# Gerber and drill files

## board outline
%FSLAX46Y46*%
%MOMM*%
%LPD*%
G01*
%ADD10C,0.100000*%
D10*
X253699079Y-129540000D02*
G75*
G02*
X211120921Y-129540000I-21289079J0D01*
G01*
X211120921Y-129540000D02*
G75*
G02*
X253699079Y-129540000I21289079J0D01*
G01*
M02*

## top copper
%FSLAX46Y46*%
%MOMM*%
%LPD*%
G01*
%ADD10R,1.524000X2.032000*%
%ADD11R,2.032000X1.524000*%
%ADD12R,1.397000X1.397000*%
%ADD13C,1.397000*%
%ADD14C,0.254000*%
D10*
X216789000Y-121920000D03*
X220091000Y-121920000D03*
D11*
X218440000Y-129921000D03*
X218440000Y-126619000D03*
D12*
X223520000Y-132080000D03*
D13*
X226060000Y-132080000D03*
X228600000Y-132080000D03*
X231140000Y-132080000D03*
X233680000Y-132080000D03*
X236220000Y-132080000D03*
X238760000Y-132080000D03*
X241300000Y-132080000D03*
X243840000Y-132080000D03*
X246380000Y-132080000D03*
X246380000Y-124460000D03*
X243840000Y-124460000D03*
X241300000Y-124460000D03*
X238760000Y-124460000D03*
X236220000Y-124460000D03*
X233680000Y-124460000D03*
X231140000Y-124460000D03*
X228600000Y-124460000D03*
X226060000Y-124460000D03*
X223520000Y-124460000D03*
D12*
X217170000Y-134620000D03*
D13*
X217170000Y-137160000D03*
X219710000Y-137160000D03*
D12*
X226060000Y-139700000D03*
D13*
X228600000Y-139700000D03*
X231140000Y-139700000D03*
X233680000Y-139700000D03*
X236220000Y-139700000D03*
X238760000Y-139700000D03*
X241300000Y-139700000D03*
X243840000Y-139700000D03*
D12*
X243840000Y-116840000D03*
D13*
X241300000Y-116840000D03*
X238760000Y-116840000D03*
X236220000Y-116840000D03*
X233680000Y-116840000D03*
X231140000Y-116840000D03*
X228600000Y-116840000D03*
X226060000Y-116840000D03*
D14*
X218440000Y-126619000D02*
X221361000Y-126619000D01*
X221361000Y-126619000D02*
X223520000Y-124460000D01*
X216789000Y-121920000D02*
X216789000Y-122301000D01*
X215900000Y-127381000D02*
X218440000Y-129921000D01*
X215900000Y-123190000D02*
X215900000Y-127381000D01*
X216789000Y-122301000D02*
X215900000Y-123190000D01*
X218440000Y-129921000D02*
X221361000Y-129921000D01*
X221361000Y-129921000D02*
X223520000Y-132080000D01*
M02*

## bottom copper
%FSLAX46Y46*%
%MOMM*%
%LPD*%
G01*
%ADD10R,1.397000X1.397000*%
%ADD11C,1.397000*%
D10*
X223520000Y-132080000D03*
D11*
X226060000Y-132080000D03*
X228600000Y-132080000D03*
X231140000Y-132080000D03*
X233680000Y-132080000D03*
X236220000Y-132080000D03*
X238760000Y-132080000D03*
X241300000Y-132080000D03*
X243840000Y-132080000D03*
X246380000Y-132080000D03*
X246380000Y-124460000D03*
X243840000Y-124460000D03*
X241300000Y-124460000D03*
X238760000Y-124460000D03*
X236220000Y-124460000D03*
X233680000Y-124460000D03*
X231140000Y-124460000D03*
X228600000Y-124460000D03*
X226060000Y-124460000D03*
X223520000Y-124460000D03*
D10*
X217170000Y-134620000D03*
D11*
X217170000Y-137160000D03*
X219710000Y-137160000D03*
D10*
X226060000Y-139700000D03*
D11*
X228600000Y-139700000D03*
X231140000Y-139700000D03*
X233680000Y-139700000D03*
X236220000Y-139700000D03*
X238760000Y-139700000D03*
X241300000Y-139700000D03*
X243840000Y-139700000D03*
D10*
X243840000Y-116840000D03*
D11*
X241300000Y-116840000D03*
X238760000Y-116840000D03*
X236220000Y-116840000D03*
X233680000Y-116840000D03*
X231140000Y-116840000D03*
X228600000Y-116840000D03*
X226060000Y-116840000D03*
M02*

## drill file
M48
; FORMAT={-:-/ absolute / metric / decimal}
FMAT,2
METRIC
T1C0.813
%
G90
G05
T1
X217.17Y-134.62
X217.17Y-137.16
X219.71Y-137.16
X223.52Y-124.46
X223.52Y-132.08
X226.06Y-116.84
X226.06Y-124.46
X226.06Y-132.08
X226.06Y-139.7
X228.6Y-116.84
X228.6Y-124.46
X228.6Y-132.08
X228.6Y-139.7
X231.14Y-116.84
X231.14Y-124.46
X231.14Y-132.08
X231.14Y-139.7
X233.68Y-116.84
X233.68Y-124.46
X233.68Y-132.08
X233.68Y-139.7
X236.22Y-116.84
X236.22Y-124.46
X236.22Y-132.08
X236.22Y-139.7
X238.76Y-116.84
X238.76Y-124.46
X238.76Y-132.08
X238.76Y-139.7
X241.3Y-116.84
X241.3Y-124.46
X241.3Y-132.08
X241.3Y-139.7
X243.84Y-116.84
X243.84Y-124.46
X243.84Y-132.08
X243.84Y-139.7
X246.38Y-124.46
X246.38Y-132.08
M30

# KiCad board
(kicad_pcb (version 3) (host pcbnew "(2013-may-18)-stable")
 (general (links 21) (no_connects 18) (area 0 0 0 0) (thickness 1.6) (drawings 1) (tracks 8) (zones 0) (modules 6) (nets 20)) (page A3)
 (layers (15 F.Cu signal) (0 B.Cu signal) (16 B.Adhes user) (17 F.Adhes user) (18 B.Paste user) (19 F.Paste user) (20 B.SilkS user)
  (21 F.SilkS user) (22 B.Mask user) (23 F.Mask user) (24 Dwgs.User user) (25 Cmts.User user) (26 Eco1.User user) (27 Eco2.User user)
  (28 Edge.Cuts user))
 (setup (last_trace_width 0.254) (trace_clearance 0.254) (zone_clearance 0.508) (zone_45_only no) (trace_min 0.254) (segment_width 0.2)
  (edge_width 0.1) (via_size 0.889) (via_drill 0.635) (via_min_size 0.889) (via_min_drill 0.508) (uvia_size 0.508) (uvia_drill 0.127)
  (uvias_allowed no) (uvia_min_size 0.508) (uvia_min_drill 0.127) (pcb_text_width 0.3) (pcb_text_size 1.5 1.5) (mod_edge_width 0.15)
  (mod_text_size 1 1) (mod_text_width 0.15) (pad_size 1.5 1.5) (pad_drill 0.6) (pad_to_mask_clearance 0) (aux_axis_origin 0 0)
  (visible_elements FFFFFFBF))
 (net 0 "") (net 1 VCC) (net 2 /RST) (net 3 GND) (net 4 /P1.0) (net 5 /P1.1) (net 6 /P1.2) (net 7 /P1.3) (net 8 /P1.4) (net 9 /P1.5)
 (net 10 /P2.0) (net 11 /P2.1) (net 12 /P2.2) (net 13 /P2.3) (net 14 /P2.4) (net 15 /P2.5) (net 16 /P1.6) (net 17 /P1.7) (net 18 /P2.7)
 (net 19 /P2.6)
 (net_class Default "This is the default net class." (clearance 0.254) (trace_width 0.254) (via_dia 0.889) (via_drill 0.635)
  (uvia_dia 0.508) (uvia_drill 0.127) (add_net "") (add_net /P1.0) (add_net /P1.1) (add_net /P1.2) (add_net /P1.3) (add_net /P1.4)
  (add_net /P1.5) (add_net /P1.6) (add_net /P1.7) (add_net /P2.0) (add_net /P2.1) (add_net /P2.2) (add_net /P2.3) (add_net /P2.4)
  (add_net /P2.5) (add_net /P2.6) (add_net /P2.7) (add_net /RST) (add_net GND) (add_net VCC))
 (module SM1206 (layer F.Cu) (at 218.44 121.92)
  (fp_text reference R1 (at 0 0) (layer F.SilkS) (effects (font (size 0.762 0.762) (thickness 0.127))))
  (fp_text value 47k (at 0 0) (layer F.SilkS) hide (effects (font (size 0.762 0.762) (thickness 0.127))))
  (pad 1 smd rect (at -1.651 0) (size 1.524 2.032) (layers F.Cu F.Paste F.Mask) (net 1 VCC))
  (pad 2 smd rect (at 1.651 0) (size 1.524 2.032) (layers F.Cu F.Paste F.Mask) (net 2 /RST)))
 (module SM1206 (layer F.Cu) (at 218.44 128.27 90)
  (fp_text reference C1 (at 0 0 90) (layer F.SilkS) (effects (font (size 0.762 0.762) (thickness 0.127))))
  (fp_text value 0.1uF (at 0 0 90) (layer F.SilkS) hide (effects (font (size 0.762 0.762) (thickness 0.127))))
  (pad 1 smd rect (at -1.651 0 90) (size 1.524 2.032) (layers F.Cu F.Paste F.Mask) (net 1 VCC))
  (pad 2 smd rect (at 1.651 0 90) (size 1.524 2.032) (layers F.Cu F.Paste F.Mask) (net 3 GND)))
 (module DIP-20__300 (layer F.Cu) (at 234.95 128.27)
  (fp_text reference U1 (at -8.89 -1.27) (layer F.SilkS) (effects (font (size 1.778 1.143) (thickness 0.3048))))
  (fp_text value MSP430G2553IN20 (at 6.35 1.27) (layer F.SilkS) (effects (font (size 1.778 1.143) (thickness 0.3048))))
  (pad 1 thru_hole rect (at -11.43 3.81) (size 1.397 1.397) (drill 0.8128) (layers *.Cu *.Mask F.SilkS) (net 1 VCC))
  (pad 2 thru_hole circle (at -8.89 3.81) (size 1.397 1.397) (drill 0.8128) (layers *.Cu *.Mask F.SilkS) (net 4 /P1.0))
  (pad 3 thru_hole circle (at -6.35 3.81) (size 1.397 1.397) (drill 0.8128) (layers *.Cu *.Mask F.SilkS) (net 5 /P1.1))
  (pad 4 thru_hole circle (at -3.81 3.81) (size 1.397 1.397) (drill 0.8128) (layers *.Cu *.Mask F.SilkS) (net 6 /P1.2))
  (pad 5 thru_hole circle (at -1.27 3.81) (size 1.397 1.397) (drill 0.8128) (layers *.Cu *.Mask F.SilkS) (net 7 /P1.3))
  (pad 6 thru_hole circle (at 1.27 3.81) (size 1.397 1.397) (drill 0.8128) (layers *.Cu *.Mask F.SilkS) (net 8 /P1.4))
  (pad 7 thru_hole circle (at 3.81 3.81) (size 1.397 1.397) (drill 0.8128) (layers *.Cu *.Mask F.SilkS) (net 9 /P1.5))
  (pad 8 thru_hole circle (at 6.35 3.81) (size 1.397 1.397) (drill 0.8128) (layers *.Cu *.Mask F.SilkS) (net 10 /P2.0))
  (pad 9 thru_hole circle (at 8.89 3.81) (size 1.397 1.397) (drill 0.8128) (layers *.Cu *.Mask F.SilkS) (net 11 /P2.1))
  (pad 10 thru_hole circle (at 11.43 3.81) (size 1.397 1.397) (drill 0.8128) (layers *.Cu *.Mask F.SilkS) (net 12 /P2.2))
  (pad 11 thru_hole circle (at 11.43 -3.81) (size 1.397 1.397) (drill 0.8128) (layers *.Cu *.Mask F.SilkS) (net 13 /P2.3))
  (pad 12 thru_hole circle (at 8.89 -3.81) (size 1.397 1.397) (drill 0.8128) (layers *.Cu *.Mask F.SilkS) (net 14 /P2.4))
  (pad 13 thru_hole circle (at 6.35 -3.81) (size 1.397 1.397) (drill 0.8128) (layers *.Cu *.Mask F.SilkS) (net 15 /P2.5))
  (pad 14 thru_hole circle (at 3.81 -3.81) (size 1.397 1.397) (drill 0.8128) (layers *.Cu *.Mask F.SilkS) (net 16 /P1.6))
  (pad 15 thru_hole circle (at 1.27 -3.81) (size 1.397 1.397) (drill 0.8128) (layers *.Cu *.Mask F.SilkS) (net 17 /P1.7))
  (pad 16 thru_hole circle (at -1.27 -3.81) (size 1.397 1.397) (drill 0.8128) (layers *.Cu *.Mask F.SilkS) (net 2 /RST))
  (pad 17 thru_hole circle (at -3.81 -3.81) (size 1.397 1.397) (drill 0.8128) (layers *.Cu *.Mask F.SilkS))
  (pad 18 thru_hole circle (at -6.35 -3.81) (size 1.397 1.397) (drill 0.8128) (layers *.Cu *.Mask F.SilkS) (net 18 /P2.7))
  (pad 19 thru_hole circle (at -8.89 -3.81) (size 1.397 1.397) (drill 0.8128) (layers *.Cu *.Mask F.SilkS) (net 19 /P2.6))
  (pad 20 thru_hole circle (at -11.43 -3.81) (size 1.397 1.397) (drill 0.8128) (layers *.Cu *.Mask F.SilkS) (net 3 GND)))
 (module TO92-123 (layer F.Cu) (at 218.44 135.89 90)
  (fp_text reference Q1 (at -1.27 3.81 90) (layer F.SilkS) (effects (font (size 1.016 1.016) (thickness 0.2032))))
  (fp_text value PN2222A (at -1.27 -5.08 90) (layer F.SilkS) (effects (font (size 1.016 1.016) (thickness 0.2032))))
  (pad 3 thru_hole rect (at 1.27 -1.27 90) (size 1.397 1.397) (drill 0.8128) (layers *.Cu *.Mask F.SilkS))
  (pad 2 thru_hole circle (at -1.27 -1.27 90) (size 1.397 1.397) (drill 0.8128) (layers *.Cu *.Mask F.SilkS) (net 4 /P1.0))
  (pad 1 thru_hole circle (at -1.27 1.27 90) (size 1.397 1.397) (drill 0.8128) (layers *.Cu *.Mask F.SilkS)))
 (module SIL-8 (layer F.Cu) (at 234.95 139.7)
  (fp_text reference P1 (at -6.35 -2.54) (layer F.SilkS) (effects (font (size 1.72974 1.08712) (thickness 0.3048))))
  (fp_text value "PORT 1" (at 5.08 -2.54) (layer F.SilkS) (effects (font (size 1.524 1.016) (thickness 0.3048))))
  (pad 1 thru_hole rect (at -8.89 0) (size 1.397 1.397) (drill 0.8128) (layers *.Cu *.Mask F.SilkS) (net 4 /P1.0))
  (pad 2 thru_hole circle (at -6.35 0) (size 1.397 1.397) (drill 0.8128) (layers *.Cu *.Mask F.SilkS) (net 5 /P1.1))
  (pad 3 thru_hole circle (at -3.81 0) (size 1.397 1.397) (drill 0.8128) (layers *.Cu *.Mask F.SilkS) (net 6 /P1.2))
  (pad 4 thru_hole circle (at -1.27 0) (size 1.397 1.397) (drill 0.8128) (layers *.Cu *.Mask F.SilkS) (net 7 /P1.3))
  (pad 5 thru_hole circle (at 1.27 0) (size 1.397 1.397) (drill 0.8128) (layers *.Cu *.Mask F.SilkS) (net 8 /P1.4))
  (pad 6 thru_hole circle (at 3.81 0) (size 1.397 1.397) (drill 0.8128) (layers *.Cu *.Mask F.SilkS) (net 9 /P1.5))
  (pad 7 thru_hole circle (at 6.35 0) (size 1.397 1.397) (drill 0.8128) (layers *.Cu *.Mask F.SilkS) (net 16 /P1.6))
  (pad 8 thru_hole circle (at 8.89 0) (size 1.397 1.397) (drill 0.8128) (layers *.Cu *.Mask F.SilkS) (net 17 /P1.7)))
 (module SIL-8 (layer F.Cu) (at 234.95 116.84 180)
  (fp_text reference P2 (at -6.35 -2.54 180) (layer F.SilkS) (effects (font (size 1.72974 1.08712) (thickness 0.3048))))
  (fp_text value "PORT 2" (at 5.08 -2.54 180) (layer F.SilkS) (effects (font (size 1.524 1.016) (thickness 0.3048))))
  (pad 1 thru_hole rect (at -8.89 0 180) (size 1.397 1.397) (drill 0.8128) (layers *.Cu *.Mask F.SilkS) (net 10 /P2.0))
  (pad 2 thru_hole circle (at -6.35 0 180) (size 1.397 1.397) (drill 0.8128) (layers *.Cu *.Mask F.SilkS) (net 11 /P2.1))
  (pad 3 thru_hole circle (at -3.81 0 180) (size 1.397 1.397) (drill 0.8128) (layers *.Cu *.Mask F.SilkS) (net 12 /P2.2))
  (pad 4 thru_hole circle (at -1.27 0 180) (size 1.397 1.397) (drill 0.8128) (layers *.Cu *.Mask F.SilkS) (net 13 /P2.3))
  (pad 5 thru_hole circle (at 1.27 0 180) (size 1.397 1.397) (drill 0.8128) (layers *.Cu *.Mask F.SilkS) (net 14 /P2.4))
  (pad 6 thru_hole circle (at 3.81 0 180) (size 1.397 1.397) (drill 0.8128) (layers *.Cu *.Mask F.SilkS) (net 15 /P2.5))
  (pad 7 thru_hole circle (at 6.35 0 180) (size 1.397 1.397) (drill 0.8128) (layers *.Cu *.Mask F.SilkS) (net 19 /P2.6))
  (pad 8 thru_hole circle (at 8.89 0 180) (size 1.397 1.397) (drill 0.8128) (layers *.Cu *.Mask F.SilkS) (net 18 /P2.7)))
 (gr_circle (center 232.41 129.54) (end 212.09 123.19) (layer Edge.Cuts) (width 0.1))
 (segment (start 218.44 126.619) (end 221.361 126.619) (width 0.254) (layer F.Cu) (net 3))
 (segment (start 221.361 126.619) (end 223.52 124.46) (width 0.254) (layer F.Cu) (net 3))
 (segment (start 216.789 121.92) (end 216.789 122.301) (width 0.254) (layer F.Cu) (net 1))
 (segment (start 215.9 127.381) (end 218.44 129.921) (width 0.254) (layer F.Cu) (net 1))
 (segment (start 215.9 123.19) (end 215.9 127.381) (width 0.254) (layer F.Cu) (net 1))
 (segment (start 216.789 122.301) (end 215.9 123.19) (width 0.254) (layer F.Cu) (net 1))
 (segment (start 218.44 129.921) (end 221.361 129.921) (width 0.254) (layer F.Cu) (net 1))
 (segment (start 221.361 129.921) (end 223.52 132.08) (width 0.254) (layer F.Cu) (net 1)))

